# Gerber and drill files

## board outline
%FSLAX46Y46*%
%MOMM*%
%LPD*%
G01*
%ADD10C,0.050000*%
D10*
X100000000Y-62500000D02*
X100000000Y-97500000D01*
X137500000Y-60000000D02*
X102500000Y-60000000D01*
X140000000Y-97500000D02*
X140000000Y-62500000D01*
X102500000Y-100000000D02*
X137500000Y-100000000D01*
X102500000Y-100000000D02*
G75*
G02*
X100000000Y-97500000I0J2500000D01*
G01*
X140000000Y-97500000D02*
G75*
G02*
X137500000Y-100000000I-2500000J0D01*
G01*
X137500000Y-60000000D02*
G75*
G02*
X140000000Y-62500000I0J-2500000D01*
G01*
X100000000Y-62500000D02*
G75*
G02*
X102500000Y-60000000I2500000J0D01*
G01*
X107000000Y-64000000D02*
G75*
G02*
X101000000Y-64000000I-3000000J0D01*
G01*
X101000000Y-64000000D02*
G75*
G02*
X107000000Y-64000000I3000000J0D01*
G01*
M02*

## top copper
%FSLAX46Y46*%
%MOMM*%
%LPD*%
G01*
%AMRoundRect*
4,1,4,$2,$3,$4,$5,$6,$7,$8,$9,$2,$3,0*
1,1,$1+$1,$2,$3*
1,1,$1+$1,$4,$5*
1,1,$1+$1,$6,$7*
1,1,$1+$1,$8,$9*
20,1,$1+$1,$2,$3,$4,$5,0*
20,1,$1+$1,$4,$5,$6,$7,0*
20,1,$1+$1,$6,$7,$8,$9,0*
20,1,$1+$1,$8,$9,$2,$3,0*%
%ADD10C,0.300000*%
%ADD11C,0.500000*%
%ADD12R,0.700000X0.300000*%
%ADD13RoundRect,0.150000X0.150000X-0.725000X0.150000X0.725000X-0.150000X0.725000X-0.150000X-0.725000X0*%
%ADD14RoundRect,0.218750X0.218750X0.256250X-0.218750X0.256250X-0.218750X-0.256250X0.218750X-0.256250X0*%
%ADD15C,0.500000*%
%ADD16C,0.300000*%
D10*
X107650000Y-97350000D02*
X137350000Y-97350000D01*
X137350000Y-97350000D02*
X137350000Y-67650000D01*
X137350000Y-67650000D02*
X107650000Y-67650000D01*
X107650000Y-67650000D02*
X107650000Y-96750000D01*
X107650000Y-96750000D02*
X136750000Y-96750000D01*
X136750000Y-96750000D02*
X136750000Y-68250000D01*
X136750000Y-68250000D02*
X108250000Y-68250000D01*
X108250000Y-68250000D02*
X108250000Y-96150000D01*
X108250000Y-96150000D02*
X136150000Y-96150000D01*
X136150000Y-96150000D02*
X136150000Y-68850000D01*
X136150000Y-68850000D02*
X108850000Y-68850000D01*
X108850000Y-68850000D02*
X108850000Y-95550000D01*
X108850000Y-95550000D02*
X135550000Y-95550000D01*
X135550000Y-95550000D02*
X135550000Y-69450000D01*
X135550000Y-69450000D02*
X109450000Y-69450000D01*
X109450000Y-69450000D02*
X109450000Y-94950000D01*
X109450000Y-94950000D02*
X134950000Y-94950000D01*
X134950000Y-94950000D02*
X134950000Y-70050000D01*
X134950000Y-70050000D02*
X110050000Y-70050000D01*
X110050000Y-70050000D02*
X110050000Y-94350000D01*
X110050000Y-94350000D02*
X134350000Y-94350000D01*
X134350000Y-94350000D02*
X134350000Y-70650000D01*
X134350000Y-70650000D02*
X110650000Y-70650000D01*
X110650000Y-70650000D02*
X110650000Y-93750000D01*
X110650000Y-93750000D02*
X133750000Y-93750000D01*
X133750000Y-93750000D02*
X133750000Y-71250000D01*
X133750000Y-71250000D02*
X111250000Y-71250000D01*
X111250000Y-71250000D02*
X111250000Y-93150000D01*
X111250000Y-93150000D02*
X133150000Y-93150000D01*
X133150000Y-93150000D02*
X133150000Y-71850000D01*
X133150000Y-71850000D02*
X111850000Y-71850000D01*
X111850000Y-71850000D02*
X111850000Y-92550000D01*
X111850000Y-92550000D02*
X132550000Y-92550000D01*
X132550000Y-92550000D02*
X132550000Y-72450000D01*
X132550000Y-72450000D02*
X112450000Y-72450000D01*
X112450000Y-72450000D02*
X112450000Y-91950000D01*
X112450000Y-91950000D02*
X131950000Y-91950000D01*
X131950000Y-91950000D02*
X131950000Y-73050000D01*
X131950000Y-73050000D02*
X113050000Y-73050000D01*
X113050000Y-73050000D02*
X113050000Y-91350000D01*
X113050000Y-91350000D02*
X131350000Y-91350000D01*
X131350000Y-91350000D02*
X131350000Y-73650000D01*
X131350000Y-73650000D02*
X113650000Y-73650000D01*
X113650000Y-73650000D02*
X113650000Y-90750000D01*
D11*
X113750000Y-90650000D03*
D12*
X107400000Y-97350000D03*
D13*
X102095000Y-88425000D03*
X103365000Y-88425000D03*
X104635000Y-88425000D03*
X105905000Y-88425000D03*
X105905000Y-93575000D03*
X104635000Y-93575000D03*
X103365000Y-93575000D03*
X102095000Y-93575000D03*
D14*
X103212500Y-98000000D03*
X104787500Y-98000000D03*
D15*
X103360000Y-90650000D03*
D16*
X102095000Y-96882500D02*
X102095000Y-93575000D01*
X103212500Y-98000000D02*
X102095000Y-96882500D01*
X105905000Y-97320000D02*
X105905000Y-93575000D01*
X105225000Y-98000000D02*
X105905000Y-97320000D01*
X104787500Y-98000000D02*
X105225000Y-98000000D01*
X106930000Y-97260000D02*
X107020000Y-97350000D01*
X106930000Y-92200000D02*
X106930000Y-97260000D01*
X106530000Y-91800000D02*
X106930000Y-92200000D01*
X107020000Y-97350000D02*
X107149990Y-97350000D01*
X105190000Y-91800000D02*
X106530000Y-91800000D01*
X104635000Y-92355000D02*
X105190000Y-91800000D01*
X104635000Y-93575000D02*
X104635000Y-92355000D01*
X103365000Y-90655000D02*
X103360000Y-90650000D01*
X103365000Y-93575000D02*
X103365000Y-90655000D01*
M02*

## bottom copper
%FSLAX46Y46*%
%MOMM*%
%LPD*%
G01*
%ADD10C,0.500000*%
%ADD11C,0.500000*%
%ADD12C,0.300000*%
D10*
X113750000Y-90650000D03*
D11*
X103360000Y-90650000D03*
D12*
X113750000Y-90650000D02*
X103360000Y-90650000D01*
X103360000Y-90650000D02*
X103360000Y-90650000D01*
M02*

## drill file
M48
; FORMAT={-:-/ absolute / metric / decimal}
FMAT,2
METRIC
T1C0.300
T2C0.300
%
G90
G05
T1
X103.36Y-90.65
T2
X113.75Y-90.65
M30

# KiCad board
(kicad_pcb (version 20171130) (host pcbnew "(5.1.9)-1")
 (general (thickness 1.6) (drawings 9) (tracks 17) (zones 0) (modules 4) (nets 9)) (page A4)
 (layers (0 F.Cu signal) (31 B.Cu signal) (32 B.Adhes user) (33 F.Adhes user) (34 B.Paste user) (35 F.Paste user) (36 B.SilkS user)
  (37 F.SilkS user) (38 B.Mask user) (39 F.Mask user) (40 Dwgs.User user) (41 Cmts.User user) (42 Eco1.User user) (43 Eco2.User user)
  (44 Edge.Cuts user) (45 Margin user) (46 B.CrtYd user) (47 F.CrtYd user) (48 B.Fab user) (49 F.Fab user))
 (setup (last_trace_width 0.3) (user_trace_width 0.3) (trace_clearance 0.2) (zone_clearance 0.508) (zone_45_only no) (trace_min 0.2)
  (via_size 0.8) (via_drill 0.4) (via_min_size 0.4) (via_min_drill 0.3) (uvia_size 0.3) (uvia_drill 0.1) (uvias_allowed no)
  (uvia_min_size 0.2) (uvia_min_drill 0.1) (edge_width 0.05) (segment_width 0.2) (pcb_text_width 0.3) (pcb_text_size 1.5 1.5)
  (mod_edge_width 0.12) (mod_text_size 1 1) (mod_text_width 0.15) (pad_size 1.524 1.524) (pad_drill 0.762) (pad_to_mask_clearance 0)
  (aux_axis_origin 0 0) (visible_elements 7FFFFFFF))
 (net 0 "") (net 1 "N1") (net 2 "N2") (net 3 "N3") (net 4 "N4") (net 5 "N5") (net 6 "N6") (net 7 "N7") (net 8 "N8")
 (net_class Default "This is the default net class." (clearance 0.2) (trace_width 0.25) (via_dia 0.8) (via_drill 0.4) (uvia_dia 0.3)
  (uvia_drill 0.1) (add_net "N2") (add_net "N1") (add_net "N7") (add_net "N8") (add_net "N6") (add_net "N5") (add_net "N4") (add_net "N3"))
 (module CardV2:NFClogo (layer F.Cu) (at 122.5 82.5)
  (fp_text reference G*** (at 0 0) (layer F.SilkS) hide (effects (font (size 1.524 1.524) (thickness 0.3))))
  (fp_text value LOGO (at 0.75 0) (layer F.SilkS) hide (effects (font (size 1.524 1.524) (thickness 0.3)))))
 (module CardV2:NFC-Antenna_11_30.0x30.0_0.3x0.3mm (layer F.Cu) (at 122.5 82.5)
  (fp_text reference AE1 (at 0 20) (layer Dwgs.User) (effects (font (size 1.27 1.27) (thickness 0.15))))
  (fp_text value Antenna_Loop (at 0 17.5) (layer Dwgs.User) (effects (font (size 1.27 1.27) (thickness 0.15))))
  (fp_line (start -14.85 14.85) (end 14.85 14.85) (layer F.Cu) (width 0.3))
  (fp_line (start 14.85 14.85) (end 14.85 -14.85) (layer F.Cu) (width 0.3))
  (fp_line (start 14.85 -14.85) (end -14.85 -14.85) (layer F.Cu) (width 0.3))
  (fp_line (start -14.85 -14.85) (end -14.85 14.25) (layer F.Cu) (width 0.3))
  (fp_line (start -14.85 14.25) (end 14.25 14.25) (layer F.Cu) (width 0.3))
  (fp_line (start 14.25 14.25) (end 14.25 -14.25) (layer F.Cu) (width 0.3))
  (fp_line (start 14.25 -14.25) (end -14.25 -14.25) (layer F.Cu) (width 0.3))
  (fp_line (start -14.25 -14.25) (end -14.25 13.65) (layer F.Cu) (width 0.3))
  (fp_line (start -14.25 13.65) (end 13.65 13.65) (layer F.Cu) (width 0.3))
  (fp_line (start 13.65 13.65) (end 13.65 -13.65) (layer F.Cu) (width 0.3))
  (fp_line (start 13.65 -13.65) (end -13.65 -13.65) (layer F.Cu) (width 0.3))
  (fp_line (start -13.65 -13.65) (end -13.65 13.05) (layer F.Cu) (width 0.3))
  (fp_line (start -13.65 13.05) (end 13.05 13.05) (layer F.Cu) (width 0.3))
  (fp_line (start 13.05 13.05) (end 13.05 -13.05) (layer F.Cu) (width 0.3))
  (fp_line (start 13.05 -13.05) (end -13.05 -13.05) (layer F.Cu) (width 0.3))
  (fp_line (start -13.05 -13.05) (end -13.05 12.45) (layer F.Cu) (width 0.3))
  (fp_line (start -13.05 12.45) (end 12.45 12.45) (layer F.Cu) (width 0.3))
  (fp_line (start 12.45 12.45) (end 12.45 -12.45) (layer F.Cu) (width 0.3))
  (fp_line (start 12.45 -12.45) (end -12.45 -12.45) (layer F.Cu) (width 0.3))
  (fp_line (start -12.45 -12.45) (end -12.45 11.85) (layer F.Cu) (width 0.3))
  (fp_line (start -12.45 11.85) (end 11.85 11.85) (layer F.Cu) (width 0.3))
  (fp_line (start 11.85 11.85) (end 11.85 -11.85) (layer F.Cu) (width 0.3))
  (fp_line (start 11.85 -11.85) (end -11.85 -11.85) (layer F.Cu) (width 0.3))
  (fp_line (start -11.85 -11.85) (end -11.85 11.25) (layer F.Cu) (width 0.3))
  (fp_line (start -11.85 11.25) (end 11.25 11.25) (layer F.Cu) (width 0.3))
  (fp_line (start 11.25 11.25) (end 11.25 -11.25) (layer F.Cu) (width 0.3))
  (fp_line (start 11.25 -11.25) (end -11.25 -11.25) (layer F.Cu) (width 0.3))
  (fp_line (start -11.25 -11.25) (end -11.25 10.65) (layer F.Cu) (width 0.3))
  (fp_line (start -11.25 10.65) (end 10.65 10.65) (layer F.Cu) (width 0.3))
  (fp_line (start 10.65 10.65) (end 10.65 -10.65) (layer F.Cu) (width 0.3))
  (fp_line (start 10.65 -10.65) (end -10.65 -10.65) (layer F.Cu) (width 0.3))
  (fp_line (start -10.65 -10.65) (end -10.65 10.05) (layer F.Cu) (width 0.3))
  (fp_line (start -10.65 10.05) (end 10.05 10.05) (layer F.Cu) (width 0.3))
  (fp_line (start 10.05 10.05) (end 10.05 -10.05) (layer F.Cu) (width 0.3))
  (fp_line (start 10.05 -10.05) (end -10.05 -10.05) (layer F.Cu) (width 0.3))
  (fp_line (start -10.05 -10.05) (end -10.05 9.45) (layer F.Cu) (width 0.3))
  (fp_line (start -10.05 9.45) (end 9.45 9.45) (layer F.Cu) (width 0.3))
  (fp_line (start 9.45 9.45) (end 9.45 -9.45) (layer F.Cu) (width 0.3))
  (fp_line (start 9.45 -9.45) (end -9.45 -9.45) (layer F.Cu) (width 0.3))
  (fp_line (start -9.45 -9.45) (end -9.45 8.85) (layer F.Cu) (width 0.3))
  (fp_line (start -9.45 8.85) (end 8.85 8.85) (layer F.Cu) (width 0.3))
  (fp_line (start 8.85 8.85) (end 8.85 -8.85) (layer F.Cu) (width 0.3))
  (fp_line (start 8.85 -8.85) (end -8.85 -8.85) (layer F.Cu) (width 0.3))
  (fp_line (start -8.85 -8.85) (end -8.85 8.25) (layer F.Cu) (width 0.3))
  (pad 2 thru_hole circle (at -8.75 8.15) (size 0.5 0.5) (drill 0.3) (layers *.Cu) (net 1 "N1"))
  (pad 1 smd rect (at -15.1 14.85) (size 0.7 0.3) (layers F.Cu) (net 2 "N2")))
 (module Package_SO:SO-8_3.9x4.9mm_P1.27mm (layer F.Cu) (at 104 91 90)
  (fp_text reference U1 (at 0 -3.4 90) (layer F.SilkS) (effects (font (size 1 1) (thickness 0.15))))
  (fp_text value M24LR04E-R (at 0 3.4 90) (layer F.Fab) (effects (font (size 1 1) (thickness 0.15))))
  (pad 8 smd roundrect (at 2.575 -1.905 90) (size 1.75 0.6) (layers F.Cu F.Paste F.Mask) (roundrect_rratio 0.25) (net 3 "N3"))
  (pad 7 smd roundrect (at 2.575 -0.635 90) (size 1.75 0.6) (layers F.Cu F.Paste F.Mask) (roundrect_rratio 0.25) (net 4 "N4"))
  (pad 6 smd roundrect (at 2.575 0.635 90) (size 1.75 0.6) (layers F.Cu F.Paste F.Mask) (roundrect_rratio 0.25) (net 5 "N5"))
  (pad 5 smd roundrect (at 2.575 1.905 90) (size 1.75 0.6) (layers F.Cu F.Paste F.Mask) (roundrect_rratio 0.25) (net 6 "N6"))
  (pad 4 smd roundrect (at -2.575 1.905 90) (size 1.75 0.6) (layers F.Cu F.Paste F.Mask) (roundrect_rratio 0.25) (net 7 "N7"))
  (pad 3 smd roundrect (at -2.575 0.635 90) (size 1.75 0.6) (layers F.Cu F.Paste F.Mask) (roundrect_rratio 0.25) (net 2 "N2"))
  (pad 2 smd roundrect (at -2.575 -0.635 90) (size 1.75 0.6) (layers F.Cu F.Paste F.Mask) (roundrect_rratio 0.25) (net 1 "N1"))
  (pad 1 smd roundrect (at -2.575 -1.905 90) (size 1.75 0.6) (layers F.Cu F.Paste F.Mask) (roundrect_rratio 0.25) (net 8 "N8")))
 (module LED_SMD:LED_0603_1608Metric (layer F.Cu) (at 104 98 180)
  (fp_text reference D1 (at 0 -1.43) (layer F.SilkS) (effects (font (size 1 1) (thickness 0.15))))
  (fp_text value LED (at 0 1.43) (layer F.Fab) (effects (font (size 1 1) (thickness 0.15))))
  (pad 2 smd roundrect (at 0.7875 0 180) (size 0.875 0.95) (layers F.Cu F.Paste F.Mask) (roundrect_rratio 0.25) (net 8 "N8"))
  (pad 1 smd roundrect (at -0.7875 0 180) (size 0.875 0.95) (layers F.Cu F.Paste F.Mask) (roundrect_rratio 0.25) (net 7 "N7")))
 (gr_line (start 100 62.5) (end 100 97.5) (layer Edge.Cuts) (width 0.05))
 (gr_line (start 137.5 60) (end 102.5 60) (layer Edge.Cuts) (width 0.05))
 (gr_line (start 140 97.5) (end 140 62.5) (layer Edge.Cuts) (width 0.05))
 (gr_line (start 102.5 100) (end 137.5 100) (layer Edge.Cuts) (width 0.05))
 (gr_arc (start 102.5 97.5) (end 100 97.5) (angle -90) (layer Edge.Cuts) (width 0.05))
 (gr_arc (start 137.5 97.5) (end 137.5 100) (angle -90) (layer Edge.Cuts) (width 0.05))
 (gr_arc (start 137.5 62.5) (end 140 62.5) (angle -90) (layer Edge.Cuts) (width 0.05))
 (gr_arc (start 102.5 62.5) (end 102.5 60) (angle -90) (layer Edge.Cuts) (width 0.05))
 (gr_circle (center 104 64) (end 107 64) (layer Edge.Cuts) (width 0.05))
 (segment (start 102.095 96.8825) (end 102.095 93.575) (width 0.3) (layer F.Cu) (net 8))
 (segment (start 103.2125 98) (end 102.095 96.8825) (width 0.3) (layer F.Cu) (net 8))
 (segment (start 105.905 97.32) (end 105.905 93.575) (width 0.3) (layer F.Cu) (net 7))
 (segment (start 105.225 98) (end 105.905 97.32) (width 0.3) (layer F.Cu) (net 7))
 (segment (start 104.7875 98) (end 105.225 98) (width 0.3) (layer F.Cu) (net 7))
 (segment (start 106.93 97.26) (end 107.02 97.35) (width 0.3) (layer F.Cu) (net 2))
 (segment (start 106.93 92.2) (end 106.93 97.26) (width 0.3) (layer F.Cu) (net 2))
 (segment (start 106.53 91.8) (end 106.93 92.2) (width 0.3) (layer F.Cu) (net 2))
 (segment (start 107.02 97.35) (end 107.14999 97.35) (width 0.3) (layer F.Cu) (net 2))
 (segment (start 105.19 91.8) (end 106.53 91.8) (width 0.3) (layer F.Cu) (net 2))
 (segment (start 104.635 92.355) (end 105.19 91.8) (width 0.3) (layer F.Cu) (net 2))
 (segment (start 104.635 93.575) (end 104.635 92.355) (width 0.3) (layer F.Cu) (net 2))
 (segment (start 113.75 90.65) (end 103.36 90.65) (width 0.3) (layer B.Cu) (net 1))
 (segment (start 103.36 90.65) (end 103.36 90.65) (width 0.3) (layer B.Cu) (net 1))
 (via blind (at 103.36 90.65) (size 0.5) (drill 0.3) (layers F.Cu B.Cu) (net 1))
 (segment (start 103.365 90.655) (end 103.36 90.65) (width 0.3) (layer F.Cu) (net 1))
 (segment (start 103.365 93.575) (end 103.365 90.655) (width 0.3) (layer F.Cu) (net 1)))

